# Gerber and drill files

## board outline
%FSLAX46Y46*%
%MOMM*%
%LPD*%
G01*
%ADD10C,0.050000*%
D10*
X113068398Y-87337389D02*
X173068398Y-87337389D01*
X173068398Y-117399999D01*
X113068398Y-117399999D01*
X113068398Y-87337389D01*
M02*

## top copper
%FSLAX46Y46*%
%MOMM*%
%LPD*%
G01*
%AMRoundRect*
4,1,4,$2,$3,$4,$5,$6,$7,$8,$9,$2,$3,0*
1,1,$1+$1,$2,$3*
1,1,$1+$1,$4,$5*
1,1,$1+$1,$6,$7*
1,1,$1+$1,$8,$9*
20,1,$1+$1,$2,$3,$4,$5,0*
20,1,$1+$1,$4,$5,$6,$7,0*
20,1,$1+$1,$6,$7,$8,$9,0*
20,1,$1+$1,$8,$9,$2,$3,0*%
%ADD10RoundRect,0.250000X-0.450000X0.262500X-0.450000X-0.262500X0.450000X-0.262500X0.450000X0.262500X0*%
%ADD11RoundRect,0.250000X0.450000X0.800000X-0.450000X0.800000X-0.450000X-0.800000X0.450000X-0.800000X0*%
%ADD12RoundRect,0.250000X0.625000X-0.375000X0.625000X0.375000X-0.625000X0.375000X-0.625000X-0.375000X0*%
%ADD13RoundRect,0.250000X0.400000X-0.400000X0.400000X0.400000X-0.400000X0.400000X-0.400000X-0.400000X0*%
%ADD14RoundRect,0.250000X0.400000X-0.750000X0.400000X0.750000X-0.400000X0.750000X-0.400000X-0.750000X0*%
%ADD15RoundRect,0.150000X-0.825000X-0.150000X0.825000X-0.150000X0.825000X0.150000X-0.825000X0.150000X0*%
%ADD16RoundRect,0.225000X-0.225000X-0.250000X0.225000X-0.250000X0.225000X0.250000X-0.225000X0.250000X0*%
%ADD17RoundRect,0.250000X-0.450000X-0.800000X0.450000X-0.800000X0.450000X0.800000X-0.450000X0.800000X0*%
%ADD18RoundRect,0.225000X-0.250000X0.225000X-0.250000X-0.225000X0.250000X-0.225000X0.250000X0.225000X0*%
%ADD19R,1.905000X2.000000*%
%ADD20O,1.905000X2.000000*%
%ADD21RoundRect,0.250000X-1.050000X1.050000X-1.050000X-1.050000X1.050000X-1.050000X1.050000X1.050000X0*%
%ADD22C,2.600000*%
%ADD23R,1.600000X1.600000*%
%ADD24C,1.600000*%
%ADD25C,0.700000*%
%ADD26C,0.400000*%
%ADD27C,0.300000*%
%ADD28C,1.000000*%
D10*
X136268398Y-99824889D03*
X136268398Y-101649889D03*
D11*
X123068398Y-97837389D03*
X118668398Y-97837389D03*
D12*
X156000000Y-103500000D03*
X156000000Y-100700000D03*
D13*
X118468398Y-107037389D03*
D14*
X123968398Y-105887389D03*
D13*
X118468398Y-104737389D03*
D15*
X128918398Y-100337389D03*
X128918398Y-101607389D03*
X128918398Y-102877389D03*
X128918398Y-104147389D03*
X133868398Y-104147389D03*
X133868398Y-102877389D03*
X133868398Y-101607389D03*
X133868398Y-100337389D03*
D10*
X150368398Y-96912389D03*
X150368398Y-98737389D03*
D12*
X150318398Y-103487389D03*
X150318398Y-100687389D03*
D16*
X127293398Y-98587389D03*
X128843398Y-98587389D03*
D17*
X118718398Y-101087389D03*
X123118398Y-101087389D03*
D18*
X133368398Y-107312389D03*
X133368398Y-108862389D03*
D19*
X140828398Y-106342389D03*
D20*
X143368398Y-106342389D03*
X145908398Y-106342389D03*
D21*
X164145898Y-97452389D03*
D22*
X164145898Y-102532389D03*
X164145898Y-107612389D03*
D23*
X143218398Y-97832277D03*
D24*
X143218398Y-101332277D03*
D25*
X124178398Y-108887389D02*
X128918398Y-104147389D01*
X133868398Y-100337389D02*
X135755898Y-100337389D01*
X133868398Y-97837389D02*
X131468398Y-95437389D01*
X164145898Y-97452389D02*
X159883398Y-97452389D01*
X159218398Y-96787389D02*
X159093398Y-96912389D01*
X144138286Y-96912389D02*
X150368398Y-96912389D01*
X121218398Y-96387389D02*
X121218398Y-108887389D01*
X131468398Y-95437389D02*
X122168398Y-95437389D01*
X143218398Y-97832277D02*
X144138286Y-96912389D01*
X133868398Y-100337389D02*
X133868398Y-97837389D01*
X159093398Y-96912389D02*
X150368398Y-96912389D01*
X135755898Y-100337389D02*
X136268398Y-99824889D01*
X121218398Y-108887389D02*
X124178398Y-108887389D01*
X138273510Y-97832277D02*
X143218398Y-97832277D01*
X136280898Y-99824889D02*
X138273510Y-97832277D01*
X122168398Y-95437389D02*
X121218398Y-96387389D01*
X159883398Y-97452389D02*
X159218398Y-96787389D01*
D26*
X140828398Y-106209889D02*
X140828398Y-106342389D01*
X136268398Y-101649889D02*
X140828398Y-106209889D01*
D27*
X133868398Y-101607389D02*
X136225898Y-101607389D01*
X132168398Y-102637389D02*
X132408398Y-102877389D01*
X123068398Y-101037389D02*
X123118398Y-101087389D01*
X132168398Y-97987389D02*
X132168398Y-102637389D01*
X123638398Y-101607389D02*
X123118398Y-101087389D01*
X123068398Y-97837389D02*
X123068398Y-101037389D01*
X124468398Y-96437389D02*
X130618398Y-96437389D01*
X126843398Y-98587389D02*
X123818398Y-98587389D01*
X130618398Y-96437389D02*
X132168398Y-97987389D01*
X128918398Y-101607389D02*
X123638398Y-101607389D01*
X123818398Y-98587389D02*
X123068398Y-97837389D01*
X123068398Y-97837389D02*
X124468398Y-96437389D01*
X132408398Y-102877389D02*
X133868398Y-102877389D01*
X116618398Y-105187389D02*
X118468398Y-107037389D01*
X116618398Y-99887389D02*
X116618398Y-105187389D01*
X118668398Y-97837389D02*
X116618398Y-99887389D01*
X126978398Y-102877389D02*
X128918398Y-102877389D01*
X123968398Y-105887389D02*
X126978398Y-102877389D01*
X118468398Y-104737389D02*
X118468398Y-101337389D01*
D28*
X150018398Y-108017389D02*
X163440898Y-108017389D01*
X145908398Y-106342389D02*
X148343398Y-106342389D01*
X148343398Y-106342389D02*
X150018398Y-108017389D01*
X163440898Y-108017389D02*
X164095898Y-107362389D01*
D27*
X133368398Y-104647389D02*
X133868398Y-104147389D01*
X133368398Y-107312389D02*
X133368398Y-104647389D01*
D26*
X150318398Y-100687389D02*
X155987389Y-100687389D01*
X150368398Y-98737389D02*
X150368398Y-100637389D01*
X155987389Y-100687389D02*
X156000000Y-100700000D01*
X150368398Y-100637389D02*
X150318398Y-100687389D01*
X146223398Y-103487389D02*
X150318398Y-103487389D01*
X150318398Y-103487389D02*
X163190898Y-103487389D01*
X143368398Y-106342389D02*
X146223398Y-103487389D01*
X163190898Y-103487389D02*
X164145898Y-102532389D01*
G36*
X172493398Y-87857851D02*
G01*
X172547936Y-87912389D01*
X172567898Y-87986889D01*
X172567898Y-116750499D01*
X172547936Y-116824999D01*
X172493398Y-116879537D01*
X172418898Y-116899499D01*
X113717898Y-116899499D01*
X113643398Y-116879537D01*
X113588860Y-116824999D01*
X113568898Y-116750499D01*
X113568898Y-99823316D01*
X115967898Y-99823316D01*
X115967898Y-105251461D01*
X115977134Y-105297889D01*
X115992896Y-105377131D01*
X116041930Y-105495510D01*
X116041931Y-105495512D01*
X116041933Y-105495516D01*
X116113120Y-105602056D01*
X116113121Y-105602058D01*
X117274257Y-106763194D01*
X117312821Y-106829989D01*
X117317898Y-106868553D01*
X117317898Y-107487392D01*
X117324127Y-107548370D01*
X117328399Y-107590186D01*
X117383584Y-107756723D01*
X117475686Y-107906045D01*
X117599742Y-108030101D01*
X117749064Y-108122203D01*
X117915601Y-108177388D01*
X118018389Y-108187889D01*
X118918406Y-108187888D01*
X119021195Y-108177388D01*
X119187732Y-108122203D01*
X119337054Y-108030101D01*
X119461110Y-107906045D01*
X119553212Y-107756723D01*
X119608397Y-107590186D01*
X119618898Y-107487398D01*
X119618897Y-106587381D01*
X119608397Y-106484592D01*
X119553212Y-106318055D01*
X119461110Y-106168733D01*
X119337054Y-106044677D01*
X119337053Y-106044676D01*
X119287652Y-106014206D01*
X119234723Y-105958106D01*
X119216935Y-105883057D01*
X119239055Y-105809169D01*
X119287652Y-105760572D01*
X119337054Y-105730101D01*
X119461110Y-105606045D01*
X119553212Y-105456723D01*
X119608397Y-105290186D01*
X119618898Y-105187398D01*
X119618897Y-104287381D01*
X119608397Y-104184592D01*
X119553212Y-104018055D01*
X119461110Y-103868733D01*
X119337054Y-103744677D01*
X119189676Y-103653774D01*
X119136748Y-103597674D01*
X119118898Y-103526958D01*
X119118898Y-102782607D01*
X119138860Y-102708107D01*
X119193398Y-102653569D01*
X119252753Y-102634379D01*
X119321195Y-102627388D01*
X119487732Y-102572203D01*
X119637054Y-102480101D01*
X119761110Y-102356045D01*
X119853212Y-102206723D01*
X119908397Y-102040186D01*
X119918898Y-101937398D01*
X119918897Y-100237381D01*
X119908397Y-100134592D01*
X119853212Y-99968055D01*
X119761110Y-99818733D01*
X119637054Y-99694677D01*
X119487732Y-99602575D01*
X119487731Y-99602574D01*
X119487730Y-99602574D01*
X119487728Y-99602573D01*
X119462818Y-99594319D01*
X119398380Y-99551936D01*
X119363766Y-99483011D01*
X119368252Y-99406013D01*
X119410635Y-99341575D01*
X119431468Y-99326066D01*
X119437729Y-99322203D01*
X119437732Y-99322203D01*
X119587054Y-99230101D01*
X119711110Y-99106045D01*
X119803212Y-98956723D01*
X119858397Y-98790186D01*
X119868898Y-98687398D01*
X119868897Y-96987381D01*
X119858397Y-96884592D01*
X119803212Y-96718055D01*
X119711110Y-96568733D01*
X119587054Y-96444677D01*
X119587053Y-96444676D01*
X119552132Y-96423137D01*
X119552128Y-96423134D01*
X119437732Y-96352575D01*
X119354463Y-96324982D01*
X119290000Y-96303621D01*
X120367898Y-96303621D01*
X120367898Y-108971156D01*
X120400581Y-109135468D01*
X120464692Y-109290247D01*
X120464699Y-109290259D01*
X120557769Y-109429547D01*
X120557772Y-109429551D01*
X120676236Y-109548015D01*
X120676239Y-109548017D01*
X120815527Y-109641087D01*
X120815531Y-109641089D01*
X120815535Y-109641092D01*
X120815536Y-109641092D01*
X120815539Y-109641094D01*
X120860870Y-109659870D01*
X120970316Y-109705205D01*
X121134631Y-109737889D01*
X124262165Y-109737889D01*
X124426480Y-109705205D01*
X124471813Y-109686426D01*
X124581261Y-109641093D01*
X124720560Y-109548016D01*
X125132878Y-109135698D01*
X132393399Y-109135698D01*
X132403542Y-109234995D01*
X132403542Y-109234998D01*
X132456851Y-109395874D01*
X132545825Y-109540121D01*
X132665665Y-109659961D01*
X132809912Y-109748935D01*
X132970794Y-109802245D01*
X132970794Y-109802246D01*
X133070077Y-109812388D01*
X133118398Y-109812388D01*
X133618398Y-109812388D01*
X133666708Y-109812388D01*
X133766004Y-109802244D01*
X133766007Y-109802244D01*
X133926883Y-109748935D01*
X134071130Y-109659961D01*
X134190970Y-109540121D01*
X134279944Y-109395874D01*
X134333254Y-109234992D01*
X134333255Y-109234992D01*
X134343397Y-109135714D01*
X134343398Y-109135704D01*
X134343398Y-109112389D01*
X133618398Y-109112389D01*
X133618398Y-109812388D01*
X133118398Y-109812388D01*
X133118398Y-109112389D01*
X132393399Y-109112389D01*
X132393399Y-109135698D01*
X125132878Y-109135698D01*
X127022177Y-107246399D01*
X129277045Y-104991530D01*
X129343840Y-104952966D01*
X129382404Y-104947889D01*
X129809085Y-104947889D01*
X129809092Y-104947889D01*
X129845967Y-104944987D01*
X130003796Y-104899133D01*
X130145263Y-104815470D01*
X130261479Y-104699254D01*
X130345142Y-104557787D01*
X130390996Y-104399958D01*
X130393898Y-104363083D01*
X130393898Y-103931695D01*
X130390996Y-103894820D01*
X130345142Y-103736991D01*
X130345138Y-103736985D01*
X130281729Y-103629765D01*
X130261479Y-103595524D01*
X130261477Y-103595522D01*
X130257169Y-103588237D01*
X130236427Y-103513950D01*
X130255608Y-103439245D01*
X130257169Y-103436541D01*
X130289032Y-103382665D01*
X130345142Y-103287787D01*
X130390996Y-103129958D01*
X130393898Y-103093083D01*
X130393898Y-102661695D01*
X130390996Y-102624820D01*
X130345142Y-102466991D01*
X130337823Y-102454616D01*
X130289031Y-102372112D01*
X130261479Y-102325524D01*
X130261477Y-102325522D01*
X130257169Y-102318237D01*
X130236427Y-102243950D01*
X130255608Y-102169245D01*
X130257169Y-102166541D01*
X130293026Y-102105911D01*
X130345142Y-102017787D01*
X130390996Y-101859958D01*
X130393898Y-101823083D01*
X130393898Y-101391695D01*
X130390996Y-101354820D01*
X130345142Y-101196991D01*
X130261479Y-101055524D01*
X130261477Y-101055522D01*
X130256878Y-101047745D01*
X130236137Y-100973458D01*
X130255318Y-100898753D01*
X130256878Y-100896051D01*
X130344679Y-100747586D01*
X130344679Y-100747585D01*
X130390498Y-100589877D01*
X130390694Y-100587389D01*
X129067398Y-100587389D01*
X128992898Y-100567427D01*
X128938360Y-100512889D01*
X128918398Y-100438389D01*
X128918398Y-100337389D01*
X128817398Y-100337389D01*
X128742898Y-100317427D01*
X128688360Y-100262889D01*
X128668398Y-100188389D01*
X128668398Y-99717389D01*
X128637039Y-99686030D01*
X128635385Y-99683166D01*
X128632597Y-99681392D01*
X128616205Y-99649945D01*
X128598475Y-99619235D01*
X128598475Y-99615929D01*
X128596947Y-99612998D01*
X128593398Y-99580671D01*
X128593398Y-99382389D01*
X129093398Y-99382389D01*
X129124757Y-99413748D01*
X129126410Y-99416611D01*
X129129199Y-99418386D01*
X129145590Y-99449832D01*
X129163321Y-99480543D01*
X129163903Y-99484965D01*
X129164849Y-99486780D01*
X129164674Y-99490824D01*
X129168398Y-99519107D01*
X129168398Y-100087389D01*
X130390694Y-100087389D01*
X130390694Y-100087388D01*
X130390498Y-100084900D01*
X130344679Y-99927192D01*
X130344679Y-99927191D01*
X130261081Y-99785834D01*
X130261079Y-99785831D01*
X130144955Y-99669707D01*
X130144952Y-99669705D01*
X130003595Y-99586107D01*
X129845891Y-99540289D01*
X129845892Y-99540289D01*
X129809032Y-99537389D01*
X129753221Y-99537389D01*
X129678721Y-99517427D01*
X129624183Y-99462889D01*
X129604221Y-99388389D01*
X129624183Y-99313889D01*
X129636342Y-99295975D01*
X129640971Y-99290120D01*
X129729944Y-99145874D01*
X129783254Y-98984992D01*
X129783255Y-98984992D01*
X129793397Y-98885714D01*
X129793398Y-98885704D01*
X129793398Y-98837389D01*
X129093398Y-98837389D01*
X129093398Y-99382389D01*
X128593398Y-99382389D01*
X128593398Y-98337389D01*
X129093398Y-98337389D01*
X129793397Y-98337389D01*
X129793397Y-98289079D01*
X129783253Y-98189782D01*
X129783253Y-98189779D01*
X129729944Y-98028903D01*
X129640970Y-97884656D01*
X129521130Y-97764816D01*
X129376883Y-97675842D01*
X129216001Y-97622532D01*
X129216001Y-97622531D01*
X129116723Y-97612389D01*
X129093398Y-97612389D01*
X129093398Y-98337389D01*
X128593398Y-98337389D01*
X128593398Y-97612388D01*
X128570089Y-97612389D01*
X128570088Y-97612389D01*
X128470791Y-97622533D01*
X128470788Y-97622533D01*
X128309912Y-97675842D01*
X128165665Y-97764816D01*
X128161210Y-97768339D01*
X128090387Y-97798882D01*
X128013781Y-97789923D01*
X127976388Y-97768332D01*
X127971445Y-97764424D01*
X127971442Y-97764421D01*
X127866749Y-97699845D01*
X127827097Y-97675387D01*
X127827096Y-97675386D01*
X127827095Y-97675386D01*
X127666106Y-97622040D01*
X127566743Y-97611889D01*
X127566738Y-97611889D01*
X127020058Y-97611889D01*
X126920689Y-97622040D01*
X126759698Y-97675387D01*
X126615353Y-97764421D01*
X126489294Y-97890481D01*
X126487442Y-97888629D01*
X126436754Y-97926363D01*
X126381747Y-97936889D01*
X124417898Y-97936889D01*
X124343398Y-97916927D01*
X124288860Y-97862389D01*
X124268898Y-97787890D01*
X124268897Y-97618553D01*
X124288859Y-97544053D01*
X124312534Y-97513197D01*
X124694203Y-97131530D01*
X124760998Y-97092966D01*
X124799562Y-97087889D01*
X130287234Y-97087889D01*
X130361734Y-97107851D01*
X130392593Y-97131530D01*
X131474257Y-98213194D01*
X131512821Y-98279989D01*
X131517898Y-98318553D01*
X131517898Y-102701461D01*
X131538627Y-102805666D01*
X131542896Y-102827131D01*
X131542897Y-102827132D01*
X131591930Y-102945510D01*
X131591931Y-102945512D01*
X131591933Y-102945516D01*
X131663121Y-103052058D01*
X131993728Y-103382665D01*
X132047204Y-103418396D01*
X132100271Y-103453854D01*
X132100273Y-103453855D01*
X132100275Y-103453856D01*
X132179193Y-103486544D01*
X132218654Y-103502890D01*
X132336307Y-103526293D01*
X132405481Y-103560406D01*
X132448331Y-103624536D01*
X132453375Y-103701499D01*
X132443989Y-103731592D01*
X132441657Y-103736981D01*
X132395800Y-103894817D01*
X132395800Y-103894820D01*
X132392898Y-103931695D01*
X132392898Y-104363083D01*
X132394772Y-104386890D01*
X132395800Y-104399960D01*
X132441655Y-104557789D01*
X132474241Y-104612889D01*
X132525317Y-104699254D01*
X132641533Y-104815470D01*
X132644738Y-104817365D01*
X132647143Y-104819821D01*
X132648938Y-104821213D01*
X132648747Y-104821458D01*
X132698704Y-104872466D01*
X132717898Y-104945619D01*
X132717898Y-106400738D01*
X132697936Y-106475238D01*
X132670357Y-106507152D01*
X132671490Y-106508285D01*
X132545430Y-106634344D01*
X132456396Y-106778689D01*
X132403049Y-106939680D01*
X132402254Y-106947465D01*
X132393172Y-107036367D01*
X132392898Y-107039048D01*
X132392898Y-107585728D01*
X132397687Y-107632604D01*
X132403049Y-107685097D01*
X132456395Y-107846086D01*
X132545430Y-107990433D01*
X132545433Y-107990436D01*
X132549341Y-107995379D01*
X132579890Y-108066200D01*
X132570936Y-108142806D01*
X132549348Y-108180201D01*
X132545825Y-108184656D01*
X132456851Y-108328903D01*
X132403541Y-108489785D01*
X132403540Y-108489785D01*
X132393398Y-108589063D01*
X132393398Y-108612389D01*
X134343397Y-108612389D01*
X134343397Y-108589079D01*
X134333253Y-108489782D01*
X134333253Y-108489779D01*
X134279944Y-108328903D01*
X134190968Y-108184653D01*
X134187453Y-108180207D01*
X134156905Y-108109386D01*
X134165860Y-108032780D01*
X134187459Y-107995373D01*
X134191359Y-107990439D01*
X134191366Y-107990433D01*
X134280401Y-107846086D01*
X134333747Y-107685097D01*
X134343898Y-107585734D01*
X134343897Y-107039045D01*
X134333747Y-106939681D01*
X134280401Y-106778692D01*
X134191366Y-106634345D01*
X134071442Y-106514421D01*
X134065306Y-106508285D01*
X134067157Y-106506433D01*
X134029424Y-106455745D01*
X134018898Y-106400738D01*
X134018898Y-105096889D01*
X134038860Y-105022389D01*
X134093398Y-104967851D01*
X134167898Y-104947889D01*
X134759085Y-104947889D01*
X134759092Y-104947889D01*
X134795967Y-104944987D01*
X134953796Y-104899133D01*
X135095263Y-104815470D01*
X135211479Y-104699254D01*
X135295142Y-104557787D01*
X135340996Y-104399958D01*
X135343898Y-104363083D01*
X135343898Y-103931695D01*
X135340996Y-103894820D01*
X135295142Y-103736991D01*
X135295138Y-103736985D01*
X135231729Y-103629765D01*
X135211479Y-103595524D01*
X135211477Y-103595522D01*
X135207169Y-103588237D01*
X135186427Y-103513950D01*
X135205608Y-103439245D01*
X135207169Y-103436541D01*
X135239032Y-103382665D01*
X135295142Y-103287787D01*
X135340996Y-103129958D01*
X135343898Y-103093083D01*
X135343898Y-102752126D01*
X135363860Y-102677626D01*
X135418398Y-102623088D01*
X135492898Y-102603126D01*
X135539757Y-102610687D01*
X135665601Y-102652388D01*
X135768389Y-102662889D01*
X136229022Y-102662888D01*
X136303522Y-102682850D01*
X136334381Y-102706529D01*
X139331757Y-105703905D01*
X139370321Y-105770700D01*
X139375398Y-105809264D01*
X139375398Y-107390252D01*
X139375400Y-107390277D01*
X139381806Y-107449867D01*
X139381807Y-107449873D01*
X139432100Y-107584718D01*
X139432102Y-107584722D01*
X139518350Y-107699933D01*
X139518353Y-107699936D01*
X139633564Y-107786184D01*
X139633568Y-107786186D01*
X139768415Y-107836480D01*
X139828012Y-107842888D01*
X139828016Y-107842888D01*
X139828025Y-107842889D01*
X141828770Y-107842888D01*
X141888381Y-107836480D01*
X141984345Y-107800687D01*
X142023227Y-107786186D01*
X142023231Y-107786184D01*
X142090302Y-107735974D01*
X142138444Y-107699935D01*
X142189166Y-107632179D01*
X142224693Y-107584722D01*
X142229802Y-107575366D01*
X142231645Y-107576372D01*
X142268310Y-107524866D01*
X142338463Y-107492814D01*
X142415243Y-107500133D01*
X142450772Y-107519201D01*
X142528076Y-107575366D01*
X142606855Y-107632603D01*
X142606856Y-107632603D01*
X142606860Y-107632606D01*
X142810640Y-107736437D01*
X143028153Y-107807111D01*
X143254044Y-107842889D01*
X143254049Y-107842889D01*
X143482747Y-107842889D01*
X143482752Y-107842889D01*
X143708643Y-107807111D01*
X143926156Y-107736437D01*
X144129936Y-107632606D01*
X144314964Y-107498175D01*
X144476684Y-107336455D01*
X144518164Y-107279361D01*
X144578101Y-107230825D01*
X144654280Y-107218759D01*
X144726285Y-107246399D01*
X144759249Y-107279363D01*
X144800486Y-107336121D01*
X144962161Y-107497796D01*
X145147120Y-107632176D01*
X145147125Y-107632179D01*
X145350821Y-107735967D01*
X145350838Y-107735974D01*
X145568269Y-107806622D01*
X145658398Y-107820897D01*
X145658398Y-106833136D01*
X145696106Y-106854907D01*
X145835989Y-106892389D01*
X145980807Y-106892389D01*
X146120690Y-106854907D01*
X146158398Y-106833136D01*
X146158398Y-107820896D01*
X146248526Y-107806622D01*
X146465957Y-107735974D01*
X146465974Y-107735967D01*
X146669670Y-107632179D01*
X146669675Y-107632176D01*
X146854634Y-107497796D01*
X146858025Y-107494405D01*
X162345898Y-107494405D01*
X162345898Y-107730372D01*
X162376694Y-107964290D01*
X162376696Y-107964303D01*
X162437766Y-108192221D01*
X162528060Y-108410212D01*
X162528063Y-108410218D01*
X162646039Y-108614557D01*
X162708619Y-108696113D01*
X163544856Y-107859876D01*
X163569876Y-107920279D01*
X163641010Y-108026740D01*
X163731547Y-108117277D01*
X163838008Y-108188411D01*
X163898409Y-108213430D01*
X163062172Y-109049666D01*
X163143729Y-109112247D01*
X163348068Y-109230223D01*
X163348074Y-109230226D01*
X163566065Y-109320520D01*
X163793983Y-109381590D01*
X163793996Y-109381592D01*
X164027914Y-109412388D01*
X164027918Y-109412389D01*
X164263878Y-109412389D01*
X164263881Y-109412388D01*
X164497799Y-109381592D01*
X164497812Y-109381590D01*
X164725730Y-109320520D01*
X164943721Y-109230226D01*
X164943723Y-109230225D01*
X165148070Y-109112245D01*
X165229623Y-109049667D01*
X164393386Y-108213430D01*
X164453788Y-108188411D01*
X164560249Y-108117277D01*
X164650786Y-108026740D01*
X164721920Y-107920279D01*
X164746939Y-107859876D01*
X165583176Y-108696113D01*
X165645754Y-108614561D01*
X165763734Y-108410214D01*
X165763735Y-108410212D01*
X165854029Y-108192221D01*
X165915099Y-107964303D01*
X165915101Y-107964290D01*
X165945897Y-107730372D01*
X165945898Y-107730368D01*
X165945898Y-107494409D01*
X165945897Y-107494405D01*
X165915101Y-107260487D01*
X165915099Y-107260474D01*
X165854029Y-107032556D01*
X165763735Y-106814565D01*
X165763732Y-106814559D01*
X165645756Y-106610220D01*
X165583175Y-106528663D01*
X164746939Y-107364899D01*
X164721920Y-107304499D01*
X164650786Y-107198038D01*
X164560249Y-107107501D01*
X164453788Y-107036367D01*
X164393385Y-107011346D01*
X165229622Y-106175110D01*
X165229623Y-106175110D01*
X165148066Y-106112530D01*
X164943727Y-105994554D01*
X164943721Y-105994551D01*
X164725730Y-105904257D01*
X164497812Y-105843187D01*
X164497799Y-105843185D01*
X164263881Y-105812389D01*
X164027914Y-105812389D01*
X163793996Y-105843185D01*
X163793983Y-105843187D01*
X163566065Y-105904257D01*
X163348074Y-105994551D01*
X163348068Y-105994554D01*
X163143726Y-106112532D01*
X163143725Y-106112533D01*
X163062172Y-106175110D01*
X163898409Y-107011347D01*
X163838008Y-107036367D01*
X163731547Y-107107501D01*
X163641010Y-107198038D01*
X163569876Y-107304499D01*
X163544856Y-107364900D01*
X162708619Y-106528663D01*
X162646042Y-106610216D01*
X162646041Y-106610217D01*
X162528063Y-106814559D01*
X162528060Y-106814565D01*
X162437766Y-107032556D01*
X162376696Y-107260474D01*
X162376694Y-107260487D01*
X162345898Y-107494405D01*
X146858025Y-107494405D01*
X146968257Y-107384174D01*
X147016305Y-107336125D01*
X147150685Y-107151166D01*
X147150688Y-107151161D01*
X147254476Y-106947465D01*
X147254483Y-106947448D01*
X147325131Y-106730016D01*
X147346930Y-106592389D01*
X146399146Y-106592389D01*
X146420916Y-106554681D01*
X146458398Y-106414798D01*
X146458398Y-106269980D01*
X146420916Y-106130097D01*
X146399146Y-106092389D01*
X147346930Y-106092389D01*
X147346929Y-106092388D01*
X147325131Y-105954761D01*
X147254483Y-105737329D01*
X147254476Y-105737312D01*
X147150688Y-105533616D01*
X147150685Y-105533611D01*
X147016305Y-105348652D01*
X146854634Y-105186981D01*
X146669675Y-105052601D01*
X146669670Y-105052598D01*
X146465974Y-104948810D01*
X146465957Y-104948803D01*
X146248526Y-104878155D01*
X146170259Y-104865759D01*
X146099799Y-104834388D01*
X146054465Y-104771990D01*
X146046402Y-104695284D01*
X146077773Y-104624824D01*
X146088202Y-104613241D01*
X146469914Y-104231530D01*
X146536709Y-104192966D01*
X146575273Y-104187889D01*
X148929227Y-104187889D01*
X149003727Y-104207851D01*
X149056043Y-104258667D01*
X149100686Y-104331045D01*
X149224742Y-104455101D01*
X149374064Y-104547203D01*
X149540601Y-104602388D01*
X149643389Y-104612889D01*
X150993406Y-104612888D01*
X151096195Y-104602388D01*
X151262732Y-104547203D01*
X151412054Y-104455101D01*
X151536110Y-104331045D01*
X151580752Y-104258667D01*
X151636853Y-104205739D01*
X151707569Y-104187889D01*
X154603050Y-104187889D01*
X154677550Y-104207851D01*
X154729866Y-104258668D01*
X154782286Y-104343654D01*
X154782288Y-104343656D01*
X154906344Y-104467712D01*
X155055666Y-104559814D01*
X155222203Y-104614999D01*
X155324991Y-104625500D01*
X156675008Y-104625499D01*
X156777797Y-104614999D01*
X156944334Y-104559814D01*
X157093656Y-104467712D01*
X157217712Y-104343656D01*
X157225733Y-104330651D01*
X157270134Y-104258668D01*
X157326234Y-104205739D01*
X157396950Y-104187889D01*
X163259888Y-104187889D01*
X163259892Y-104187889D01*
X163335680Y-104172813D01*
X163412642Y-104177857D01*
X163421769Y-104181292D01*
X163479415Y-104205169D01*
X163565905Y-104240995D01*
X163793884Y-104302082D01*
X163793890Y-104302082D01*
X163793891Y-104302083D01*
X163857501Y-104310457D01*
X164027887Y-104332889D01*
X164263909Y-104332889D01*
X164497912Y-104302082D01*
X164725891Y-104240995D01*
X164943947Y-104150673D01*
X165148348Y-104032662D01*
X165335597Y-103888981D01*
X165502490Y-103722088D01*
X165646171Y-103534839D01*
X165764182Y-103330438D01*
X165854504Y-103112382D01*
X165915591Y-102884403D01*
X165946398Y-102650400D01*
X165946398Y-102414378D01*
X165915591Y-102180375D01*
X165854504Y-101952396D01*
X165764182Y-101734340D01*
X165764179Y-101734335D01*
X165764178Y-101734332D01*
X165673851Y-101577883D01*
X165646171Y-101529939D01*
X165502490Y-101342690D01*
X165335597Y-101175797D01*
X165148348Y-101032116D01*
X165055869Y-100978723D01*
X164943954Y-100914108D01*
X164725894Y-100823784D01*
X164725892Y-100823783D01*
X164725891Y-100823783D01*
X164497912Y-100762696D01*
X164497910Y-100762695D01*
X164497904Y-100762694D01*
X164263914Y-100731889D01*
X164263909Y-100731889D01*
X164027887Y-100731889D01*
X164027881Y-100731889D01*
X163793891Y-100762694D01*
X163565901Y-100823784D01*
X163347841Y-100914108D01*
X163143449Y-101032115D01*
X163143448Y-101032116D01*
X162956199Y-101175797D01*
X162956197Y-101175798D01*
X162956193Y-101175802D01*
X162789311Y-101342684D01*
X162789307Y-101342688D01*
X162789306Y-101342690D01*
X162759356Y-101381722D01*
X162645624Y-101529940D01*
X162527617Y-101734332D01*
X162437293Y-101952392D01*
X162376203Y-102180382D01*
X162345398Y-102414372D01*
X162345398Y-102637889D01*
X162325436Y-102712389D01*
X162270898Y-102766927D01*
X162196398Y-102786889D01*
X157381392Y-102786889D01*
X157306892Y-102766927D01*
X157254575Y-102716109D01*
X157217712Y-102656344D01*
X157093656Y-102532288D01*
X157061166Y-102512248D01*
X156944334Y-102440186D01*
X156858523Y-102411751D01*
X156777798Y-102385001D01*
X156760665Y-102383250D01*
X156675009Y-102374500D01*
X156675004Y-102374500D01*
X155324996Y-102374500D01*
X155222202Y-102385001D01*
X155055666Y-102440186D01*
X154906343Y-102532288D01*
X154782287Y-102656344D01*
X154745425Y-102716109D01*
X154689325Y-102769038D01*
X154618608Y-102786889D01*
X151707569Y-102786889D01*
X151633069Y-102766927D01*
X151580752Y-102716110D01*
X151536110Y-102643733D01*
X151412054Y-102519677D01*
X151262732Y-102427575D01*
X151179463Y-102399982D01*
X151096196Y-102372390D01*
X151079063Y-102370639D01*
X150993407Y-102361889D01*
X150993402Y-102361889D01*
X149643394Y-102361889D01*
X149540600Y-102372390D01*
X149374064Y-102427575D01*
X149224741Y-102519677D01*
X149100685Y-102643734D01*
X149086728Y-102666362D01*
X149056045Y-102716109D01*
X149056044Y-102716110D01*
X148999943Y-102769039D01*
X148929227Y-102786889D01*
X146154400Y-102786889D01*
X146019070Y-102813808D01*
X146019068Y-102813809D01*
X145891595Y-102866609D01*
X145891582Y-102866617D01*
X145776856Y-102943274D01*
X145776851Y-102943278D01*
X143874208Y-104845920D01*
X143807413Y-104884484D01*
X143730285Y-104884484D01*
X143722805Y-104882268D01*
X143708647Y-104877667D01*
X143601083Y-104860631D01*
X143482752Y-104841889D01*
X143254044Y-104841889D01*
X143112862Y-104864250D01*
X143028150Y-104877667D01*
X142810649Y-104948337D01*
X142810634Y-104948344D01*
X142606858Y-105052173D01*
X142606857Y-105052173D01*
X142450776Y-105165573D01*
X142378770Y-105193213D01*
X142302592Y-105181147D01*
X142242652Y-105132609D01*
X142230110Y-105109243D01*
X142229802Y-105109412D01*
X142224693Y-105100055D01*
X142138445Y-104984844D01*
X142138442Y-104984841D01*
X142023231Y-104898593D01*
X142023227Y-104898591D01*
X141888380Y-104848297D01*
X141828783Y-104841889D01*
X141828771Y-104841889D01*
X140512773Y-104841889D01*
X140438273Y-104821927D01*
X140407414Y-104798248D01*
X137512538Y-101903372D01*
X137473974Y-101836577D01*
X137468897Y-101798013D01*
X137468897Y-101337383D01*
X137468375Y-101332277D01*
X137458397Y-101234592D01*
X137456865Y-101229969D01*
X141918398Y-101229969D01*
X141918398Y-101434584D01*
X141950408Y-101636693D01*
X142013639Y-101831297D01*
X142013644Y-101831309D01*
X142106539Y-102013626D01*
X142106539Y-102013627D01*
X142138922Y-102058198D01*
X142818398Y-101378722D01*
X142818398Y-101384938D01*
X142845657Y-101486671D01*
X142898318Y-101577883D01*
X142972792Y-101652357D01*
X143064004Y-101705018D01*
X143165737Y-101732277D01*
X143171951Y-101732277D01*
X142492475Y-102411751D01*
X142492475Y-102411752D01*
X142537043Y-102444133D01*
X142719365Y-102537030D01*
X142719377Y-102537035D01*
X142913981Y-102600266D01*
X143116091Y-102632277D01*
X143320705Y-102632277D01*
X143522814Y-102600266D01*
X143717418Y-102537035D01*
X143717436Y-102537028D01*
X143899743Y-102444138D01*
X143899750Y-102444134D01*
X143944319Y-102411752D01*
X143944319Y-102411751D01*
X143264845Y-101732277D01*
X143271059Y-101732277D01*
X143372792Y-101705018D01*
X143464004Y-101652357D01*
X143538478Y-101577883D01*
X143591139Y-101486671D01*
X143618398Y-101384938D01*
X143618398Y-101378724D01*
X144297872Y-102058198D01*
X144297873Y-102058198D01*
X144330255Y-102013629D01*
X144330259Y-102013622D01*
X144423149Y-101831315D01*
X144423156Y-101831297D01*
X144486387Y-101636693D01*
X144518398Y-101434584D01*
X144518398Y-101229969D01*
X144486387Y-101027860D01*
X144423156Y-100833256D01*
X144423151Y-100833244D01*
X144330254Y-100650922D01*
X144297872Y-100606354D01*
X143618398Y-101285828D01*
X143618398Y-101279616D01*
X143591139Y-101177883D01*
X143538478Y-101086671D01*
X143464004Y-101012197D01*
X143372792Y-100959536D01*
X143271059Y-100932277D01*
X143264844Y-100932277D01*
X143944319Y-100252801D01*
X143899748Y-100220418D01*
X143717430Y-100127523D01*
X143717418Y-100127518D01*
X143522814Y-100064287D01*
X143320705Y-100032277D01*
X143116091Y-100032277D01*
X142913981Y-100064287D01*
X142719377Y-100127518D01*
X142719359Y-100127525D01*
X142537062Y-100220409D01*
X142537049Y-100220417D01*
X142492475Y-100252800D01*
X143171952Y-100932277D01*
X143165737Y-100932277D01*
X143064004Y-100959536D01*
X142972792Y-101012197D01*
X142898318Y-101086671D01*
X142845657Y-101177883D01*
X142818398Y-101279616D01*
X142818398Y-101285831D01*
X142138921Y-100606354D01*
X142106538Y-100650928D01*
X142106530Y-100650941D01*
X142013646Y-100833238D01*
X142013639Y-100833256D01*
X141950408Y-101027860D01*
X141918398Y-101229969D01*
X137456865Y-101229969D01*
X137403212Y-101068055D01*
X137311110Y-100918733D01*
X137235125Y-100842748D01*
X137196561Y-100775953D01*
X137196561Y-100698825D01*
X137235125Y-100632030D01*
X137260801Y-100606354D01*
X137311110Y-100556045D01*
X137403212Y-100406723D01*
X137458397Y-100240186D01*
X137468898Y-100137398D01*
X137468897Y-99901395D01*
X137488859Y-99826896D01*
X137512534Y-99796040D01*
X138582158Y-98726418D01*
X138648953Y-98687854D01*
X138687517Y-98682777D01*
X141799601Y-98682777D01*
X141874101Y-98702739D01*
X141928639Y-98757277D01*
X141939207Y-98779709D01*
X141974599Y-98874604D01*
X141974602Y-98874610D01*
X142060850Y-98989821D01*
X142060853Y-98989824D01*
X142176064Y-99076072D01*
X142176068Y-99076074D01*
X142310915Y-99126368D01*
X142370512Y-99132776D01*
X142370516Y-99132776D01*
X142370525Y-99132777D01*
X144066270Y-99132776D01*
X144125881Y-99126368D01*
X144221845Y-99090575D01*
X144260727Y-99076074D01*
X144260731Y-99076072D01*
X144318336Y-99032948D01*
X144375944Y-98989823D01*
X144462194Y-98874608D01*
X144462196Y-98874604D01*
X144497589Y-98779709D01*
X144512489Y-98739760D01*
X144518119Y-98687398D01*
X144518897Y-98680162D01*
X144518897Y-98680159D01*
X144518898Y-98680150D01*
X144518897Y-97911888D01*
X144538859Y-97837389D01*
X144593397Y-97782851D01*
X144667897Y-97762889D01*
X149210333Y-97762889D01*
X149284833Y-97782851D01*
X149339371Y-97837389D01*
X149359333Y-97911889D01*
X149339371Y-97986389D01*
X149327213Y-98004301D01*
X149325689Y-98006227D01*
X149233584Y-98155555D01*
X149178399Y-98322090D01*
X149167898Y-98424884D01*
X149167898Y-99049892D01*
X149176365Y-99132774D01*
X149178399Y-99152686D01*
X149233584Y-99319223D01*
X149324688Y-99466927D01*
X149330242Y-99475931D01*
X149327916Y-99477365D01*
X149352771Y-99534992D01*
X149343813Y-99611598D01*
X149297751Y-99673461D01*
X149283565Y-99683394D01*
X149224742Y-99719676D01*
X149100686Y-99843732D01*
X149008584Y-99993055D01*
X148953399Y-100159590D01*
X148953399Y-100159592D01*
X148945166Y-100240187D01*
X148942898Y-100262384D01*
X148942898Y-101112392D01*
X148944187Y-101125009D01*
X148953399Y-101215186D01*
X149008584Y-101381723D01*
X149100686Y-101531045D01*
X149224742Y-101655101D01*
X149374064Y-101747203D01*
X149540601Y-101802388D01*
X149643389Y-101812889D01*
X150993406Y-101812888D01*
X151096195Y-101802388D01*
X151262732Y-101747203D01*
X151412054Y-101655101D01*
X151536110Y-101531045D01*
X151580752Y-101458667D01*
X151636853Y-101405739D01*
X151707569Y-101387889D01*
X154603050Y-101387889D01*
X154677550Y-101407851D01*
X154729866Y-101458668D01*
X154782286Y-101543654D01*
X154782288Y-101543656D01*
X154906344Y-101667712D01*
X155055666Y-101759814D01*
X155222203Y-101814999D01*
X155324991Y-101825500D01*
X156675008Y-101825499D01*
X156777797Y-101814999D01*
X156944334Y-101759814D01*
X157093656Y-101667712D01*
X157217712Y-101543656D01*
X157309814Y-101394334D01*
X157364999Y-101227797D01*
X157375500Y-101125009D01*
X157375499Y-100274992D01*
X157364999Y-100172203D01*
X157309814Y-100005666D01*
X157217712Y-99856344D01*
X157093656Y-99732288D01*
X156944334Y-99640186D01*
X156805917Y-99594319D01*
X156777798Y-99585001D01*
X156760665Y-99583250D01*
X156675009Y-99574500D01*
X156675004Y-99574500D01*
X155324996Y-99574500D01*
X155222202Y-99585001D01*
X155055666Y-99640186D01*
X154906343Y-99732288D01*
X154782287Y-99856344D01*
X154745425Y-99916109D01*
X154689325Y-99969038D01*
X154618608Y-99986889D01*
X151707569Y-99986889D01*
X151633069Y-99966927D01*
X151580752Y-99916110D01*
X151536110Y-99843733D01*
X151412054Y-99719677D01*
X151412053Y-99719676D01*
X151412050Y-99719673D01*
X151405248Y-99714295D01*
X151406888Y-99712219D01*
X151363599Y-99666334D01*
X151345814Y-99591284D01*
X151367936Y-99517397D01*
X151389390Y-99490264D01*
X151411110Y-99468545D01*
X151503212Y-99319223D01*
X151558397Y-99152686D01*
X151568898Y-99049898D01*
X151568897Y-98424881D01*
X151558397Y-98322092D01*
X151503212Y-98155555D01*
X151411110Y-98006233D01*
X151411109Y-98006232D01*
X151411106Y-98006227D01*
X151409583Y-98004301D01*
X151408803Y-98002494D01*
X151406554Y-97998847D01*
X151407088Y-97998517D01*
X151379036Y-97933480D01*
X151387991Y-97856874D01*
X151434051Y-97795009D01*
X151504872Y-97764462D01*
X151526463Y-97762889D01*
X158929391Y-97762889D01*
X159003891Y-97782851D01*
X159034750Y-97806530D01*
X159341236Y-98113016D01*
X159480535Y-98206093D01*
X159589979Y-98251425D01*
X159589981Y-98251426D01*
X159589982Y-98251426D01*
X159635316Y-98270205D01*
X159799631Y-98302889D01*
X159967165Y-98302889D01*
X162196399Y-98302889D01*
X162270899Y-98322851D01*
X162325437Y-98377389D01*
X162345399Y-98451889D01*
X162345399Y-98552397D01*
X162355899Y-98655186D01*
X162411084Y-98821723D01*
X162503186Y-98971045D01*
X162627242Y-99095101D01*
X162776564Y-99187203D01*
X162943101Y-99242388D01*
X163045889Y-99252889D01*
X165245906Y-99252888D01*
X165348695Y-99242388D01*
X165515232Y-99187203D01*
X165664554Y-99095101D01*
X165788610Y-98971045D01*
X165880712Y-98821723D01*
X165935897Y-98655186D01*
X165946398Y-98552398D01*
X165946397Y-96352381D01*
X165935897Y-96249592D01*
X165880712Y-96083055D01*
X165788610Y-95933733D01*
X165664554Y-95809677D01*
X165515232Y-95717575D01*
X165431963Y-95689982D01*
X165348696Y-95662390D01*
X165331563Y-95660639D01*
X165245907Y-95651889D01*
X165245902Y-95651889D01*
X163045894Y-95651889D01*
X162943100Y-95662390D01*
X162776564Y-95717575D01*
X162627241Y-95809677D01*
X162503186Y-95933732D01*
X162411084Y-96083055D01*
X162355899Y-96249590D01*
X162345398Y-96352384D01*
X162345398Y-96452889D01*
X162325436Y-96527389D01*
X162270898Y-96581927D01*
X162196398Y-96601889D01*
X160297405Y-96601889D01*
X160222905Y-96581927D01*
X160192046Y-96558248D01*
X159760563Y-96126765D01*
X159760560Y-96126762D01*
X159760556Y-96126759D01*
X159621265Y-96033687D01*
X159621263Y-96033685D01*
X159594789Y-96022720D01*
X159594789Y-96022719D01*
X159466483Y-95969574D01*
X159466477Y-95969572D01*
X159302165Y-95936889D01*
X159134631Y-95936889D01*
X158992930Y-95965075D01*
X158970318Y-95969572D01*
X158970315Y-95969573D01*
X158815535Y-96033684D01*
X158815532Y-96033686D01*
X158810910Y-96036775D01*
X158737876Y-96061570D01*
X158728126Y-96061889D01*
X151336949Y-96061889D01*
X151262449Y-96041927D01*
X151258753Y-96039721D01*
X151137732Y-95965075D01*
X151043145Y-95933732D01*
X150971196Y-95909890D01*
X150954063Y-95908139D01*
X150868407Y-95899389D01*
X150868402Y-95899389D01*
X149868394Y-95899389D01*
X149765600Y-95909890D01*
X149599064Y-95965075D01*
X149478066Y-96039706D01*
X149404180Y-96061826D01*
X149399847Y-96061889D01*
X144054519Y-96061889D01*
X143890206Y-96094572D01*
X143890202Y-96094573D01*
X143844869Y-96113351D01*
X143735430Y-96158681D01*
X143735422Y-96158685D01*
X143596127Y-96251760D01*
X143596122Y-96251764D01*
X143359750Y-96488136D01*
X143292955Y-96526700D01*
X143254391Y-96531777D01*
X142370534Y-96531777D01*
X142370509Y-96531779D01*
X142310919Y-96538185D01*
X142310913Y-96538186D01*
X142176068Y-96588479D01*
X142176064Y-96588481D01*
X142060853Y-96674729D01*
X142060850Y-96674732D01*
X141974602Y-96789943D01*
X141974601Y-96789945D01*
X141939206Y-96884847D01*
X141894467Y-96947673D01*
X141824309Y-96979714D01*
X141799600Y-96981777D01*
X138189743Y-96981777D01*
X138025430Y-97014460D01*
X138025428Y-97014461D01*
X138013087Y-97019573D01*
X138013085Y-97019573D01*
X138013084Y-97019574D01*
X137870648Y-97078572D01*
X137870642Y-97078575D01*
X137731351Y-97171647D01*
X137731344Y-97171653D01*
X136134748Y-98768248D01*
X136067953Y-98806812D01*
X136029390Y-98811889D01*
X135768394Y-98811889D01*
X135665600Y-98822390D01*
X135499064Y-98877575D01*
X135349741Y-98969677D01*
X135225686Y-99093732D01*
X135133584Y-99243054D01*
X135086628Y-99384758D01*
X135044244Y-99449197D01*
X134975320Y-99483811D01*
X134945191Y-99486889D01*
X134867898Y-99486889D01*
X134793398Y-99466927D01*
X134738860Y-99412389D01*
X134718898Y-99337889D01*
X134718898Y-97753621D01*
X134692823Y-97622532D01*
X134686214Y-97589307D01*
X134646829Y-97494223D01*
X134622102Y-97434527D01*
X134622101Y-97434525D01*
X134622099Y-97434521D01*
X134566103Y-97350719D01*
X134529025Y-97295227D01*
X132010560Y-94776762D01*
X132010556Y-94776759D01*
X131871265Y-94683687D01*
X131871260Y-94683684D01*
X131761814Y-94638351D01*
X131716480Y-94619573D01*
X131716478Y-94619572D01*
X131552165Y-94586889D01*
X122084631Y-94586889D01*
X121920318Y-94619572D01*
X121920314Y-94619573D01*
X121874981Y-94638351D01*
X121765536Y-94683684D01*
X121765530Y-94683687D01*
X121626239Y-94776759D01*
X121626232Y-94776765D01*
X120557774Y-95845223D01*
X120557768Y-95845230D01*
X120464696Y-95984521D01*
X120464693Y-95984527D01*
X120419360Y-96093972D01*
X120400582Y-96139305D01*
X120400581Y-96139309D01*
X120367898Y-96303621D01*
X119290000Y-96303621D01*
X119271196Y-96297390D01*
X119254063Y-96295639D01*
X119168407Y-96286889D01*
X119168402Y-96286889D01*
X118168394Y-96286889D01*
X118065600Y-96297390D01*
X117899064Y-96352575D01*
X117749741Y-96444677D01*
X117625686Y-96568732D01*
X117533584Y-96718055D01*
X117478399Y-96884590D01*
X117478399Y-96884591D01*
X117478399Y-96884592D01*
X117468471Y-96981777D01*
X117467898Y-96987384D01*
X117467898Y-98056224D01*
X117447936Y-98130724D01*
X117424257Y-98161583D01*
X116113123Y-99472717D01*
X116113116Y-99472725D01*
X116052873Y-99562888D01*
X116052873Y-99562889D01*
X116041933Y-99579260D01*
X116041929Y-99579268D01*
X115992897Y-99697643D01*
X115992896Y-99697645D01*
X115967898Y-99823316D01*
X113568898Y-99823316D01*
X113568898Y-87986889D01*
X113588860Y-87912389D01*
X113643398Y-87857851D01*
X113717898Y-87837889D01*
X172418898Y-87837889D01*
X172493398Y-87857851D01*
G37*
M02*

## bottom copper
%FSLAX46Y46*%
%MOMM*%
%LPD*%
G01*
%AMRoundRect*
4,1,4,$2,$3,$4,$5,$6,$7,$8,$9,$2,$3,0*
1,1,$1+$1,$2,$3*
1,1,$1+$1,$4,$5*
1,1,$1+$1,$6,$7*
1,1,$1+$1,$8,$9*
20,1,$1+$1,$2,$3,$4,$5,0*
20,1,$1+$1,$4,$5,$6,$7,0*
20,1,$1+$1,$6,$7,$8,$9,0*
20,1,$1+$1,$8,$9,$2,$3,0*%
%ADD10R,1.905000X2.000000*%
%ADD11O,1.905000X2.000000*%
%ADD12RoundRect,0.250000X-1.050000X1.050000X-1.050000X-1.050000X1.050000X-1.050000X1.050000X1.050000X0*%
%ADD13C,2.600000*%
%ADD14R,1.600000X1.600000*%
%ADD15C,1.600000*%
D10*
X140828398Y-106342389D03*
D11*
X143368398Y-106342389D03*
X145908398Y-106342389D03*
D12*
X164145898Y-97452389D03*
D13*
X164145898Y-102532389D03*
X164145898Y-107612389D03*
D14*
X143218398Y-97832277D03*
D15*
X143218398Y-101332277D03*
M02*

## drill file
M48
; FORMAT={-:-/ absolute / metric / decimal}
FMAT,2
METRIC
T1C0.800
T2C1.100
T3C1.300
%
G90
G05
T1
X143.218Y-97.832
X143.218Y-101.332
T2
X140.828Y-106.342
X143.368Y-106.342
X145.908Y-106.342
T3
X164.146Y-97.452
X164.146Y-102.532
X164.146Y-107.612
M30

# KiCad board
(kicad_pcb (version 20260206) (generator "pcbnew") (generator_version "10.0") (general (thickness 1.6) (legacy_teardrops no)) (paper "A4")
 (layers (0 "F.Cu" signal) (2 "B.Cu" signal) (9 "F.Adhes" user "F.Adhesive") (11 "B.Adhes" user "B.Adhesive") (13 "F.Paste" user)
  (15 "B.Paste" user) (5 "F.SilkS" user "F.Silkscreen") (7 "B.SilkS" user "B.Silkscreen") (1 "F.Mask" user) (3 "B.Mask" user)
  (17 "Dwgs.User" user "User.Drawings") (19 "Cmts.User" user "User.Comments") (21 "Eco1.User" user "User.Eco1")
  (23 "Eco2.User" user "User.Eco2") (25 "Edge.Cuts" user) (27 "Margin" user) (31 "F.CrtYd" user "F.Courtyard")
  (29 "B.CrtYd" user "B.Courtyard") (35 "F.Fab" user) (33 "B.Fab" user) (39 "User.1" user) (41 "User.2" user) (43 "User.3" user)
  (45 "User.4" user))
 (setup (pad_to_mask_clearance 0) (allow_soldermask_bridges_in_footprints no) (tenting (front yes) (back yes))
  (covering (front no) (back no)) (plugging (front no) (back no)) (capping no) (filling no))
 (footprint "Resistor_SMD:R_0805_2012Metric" (layer "F.Cu") (at 136.268398 100.737389 -90)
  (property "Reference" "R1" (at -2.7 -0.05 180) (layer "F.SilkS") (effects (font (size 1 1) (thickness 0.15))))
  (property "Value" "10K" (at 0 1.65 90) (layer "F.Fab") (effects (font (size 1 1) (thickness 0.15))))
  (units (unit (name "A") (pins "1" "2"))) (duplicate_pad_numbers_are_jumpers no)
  (pad "1" smd roundrect (at -0.9125 0 270) (size 1.025 1.4) (layers "F.Cu" "F.Mask" "F.Paste") (roundrect_rratio 0.243902) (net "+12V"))
  (pad "2" smd roundrect (at 0.9125 0 270) (size 1.025 1.4) (layers "F.Cu" "F.Mask" "F.Paste") (roundrect_rratio 0.243902)
   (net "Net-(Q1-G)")))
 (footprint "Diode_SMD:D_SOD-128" (layer "F.Cu") (at 120.868398 97.837389 180)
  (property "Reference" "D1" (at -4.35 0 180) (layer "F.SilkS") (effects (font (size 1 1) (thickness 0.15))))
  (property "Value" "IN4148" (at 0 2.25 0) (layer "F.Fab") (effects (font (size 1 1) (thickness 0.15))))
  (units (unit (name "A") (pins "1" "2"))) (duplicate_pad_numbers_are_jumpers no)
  (pad "1" smd roundrect (at -2.2 0 180) (size 1.4 2.1) (layers "F.Cu" "F.Mask" "F.Paste") (roundrect_rratio 0.1785714286) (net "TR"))
  (pad "2" smd roundrect (at 2.2 0 180) (size 1.4 2.1) (layers "F.Cu" "F.Mask" "F.Paste") (roundrect_rratio 0.1785714286) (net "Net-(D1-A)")))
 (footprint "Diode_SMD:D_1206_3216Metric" (layer "F.Cu") (at 156 102.1 90)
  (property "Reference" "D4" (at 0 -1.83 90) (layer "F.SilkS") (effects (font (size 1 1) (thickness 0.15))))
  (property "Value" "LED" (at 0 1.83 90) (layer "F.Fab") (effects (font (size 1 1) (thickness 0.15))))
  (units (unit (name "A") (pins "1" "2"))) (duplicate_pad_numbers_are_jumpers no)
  (pad "1" smd roundrect (at -1.4 0 90) (size 1.25 1.75) (layers "F.Cu" "F.Mask" "F.Paste") (roundrect_rratio 0.2) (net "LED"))
  (pad "2" smd roundrect (at 1.4 0 90) (size 1.25 1.75) (layers "F.Cu" "F.Mask" "F.Paste") (roundrect_rratio 0.2) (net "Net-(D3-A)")))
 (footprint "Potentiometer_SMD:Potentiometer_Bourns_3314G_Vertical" (layer "F.Cu") (at 121.218398 105.887389 90)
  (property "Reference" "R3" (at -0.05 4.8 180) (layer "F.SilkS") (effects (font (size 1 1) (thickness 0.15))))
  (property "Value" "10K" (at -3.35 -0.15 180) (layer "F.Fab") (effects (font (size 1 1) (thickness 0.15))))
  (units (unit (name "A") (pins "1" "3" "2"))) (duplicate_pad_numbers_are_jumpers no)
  (pad "1" smd roundrect (at -1.15 -2.75 90) (size 1.3 1.3) (layers "F.Cu" "F.Mask" "F.Paste") (roundrect_rratio 0.1923076923)
   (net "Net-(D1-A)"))
  (pad "2" smd roundrect (at 0 2.75 90) (size 2 1.3) (layers "F.Cu" "F.Mask" "F.Paste") (roundrect_rratio 0.1923076923) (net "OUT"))
  (pad "3" smd roundrect (at 1.15 -2.75 90) (size 1.3 1.3) (layers "F.Cu" "F.Mask" "F.Paste") (roundrect_rratio 0.1923076923)
   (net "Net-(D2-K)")))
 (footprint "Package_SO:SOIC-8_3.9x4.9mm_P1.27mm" (layer "F.Cu") (at 131.393398 102.242389)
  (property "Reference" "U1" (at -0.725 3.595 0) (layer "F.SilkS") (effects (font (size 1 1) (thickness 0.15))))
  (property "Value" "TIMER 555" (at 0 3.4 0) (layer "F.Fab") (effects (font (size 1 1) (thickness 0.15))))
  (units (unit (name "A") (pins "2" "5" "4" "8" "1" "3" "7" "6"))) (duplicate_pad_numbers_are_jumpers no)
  (pad "1" smd roundrect (at -2.475 -1.905) (size 1.95 0.6) (layers "F.Cu" "F.Mask" "F.Paste") (roundrect_rratio 0.25) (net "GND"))
  (pad "2" smd roundrect (at -2.475 -0.635) (size 1.95 0.6) (layers "F.Cu" "F.Mask" "F.Paste") (roundrect_rratio 0.25) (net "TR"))
  (pad "3" smd roundrect (at -2.475 0.635) (size 1.95 0.6) (layers "F.Cu" "F.Mask" "F.Paste") (roundrect_rratio 0.25) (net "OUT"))
  (pad "4" smd roundrect (at -2.475 1.905) (size 1.95 0.6) (layers "F.Cu" "F.Mask" "F.Paste") (roundrect_rratio 0.25) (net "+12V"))
  (pad "5" smd roundrect (at 2.475 1.905) (size 1.95 0.6) (layers "F.Cu" "F.Mask" "F.Paste") (roundrect_rratio 0.25) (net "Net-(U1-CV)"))
  (pad "6" smd roundrect (at 2.475 0.635) (size 1.95 0.6) (layers "F.Cu" "F.Mask" "F.Paste") (roundrect_rratio 0.25) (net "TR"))
  (pad "7" smd roundrect (at 2.475 -0.635) (size 1.95 0.6) (layers "F.Cu" "F.Mask" "F.Paste") (roundrect_rratio 0.25) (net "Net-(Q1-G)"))
  (pad "8" smd roundrect (at 2.475 -1.905) (size 1.95 0.6) (layers "F.Cu" "F.Mask" "F.Paste") (roundrect_rratio 0.25) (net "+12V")))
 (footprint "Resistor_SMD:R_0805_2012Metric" (layer "F.Cu") (at 150.368398 97.824889 -90)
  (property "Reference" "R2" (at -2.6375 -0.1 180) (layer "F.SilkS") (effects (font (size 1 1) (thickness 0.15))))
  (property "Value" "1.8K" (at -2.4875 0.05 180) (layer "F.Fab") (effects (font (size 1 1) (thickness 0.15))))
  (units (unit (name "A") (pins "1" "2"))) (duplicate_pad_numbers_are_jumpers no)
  (pad "1" smd roundrect (at -0.9125 0 270) (size 1.025 1.4) (layers "F.Cu" "F.Mask" "F.Paste") (roundrect_rratio 0.243902) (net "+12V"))
  (pad "2" smd roundrect (at 0.9125 0 270) (size 1.025 1.4) (layers "F.Cu" "F.Mask" "F.Paste") (roundrect_rratio 0.243902)
   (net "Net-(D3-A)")))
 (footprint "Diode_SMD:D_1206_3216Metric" (layer "F.Cu") (at 150.318398 102.087389 90)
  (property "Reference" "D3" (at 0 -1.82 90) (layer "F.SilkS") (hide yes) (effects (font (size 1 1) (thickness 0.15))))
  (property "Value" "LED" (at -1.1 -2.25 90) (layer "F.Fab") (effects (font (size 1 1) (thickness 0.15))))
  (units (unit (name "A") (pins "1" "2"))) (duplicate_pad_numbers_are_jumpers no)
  (pad "1" smd roundrect (at -1.4 0 90) (size 1.25 1.75) (layers "F.Cu" "F.Mask" "F.Paste") (roundrect_rratio 0.2) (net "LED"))
  (pad "2" smd roundrect (at 1.4 0 90) (size 1.25 1.75) (layers "F.Cu" "F.Mask" "F.Paste") (roundrect_rratio 0.2) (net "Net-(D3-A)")))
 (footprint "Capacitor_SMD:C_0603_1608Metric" (layer "F.Cu") (at 128.068398 98.587389)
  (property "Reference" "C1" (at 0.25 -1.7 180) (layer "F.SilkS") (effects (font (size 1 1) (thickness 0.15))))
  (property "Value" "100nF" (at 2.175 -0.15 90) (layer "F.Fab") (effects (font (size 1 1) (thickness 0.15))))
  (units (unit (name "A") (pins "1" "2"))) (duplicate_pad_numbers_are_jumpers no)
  (pad "1" smd roundrect (at -0.775 0) (size 0.9 0.95) (layers "F.Cu" "F.Mask" "F.Paste") (roundrect_rratio 0.25) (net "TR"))
  (pad "2" smd roundrect (at 0.775 0) (size 0.9 0.95) (layers "F.Cu" "F.Mask" "F.Paste") (roundrect_rratio 0.25) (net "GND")))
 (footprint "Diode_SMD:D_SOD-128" (layer "F.Cu") (at 120.918398 101.087389)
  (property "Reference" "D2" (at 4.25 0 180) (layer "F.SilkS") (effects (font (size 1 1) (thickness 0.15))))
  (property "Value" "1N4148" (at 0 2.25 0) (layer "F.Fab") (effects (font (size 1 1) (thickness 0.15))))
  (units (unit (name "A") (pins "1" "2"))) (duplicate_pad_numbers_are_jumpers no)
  (pad "1" smd roundrect (at -2.2 0) (size 1.4 2.1) (layers "F.Cu" "F.Mask" "F.Paste") (roundrect_rratio 0.1785714286) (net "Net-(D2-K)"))
  (pad "2" smd roundrect (at 2.2 0) (size 1.4 2.1) (layers "F.Cu" "F.Mask" "F.Paste") (roundrect_rratio 0.1785714286) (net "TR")))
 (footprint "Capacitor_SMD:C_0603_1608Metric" (layer "F.Cu") (at 133.368398 108.087389 -90)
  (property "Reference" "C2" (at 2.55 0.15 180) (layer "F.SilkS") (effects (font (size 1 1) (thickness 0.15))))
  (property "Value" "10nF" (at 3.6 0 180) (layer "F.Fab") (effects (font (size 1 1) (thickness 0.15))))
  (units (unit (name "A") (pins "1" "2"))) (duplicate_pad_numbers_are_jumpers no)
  (pad "1" smd roundrect (at -0.775 0 270) (size 0.9 0.95) (layers "F.Cu" "F.Mask" "F.Paste") (roundrect_rratio 0.25) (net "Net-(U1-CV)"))
  (pad "2" smd roundrect (at 0.775 0 270) (size 0.9 0.95) (layers "F.Cu" "F.Mask" "F.Paste") (roundrect_rratio 0.25) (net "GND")))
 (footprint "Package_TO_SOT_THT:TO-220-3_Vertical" (layer "B.Cu") (at 140.828398 106.342389)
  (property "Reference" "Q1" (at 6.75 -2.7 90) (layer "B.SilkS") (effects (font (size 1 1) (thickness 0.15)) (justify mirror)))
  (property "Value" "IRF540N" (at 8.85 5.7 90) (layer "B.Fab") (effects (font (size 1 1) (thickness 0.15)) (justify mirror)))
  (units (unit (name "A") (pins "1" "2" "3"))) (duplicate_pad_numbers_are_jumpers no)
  (pad "1" thru_hole rect (at 0 0) (size 1.905 2) (drill 1.1) (layers "*.Cu" "*.Mask") (remove_unused_layers no) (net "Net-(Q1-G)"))
  (pad "2" thru_hole oval (at 2.54 0) (size 1.905 2) (drill 1.1) (layers "*.Cu" "*.Mask") (remove_unused_layers no) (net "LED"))
  (pad "3" thru_hole oval (at 5.08 0) (size 1.905 2) (drill 1.1) (layers "*.Cu" "*.Mask") (remove_unused_layers no) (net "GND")))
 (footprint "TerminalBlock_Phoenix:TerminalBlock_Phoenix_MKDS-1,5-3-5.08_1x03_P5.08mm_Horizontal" (layer "B.Cu")
  (at 164.145898 97.452389 -90)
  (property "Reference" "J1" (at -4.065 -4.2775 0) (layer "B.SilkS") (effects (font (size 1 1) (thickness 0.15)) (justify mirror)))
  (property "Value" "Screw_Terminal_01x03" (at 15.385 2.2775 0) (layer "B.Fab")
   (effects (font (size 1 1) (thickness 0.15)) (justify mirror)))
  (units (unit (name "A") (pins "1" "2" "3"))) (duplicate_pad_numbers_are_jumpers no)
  (pad "1" thru_hole roundrect (at 0 0 270) (size 2.6 2.6) (drill 1.3) (layers "*.Cu" "*.Mask") (remove_unused_layers no)
   (roundrect_rratio 0.096154) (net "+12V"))
  (pad "2" thru_hole circle (at 5.08 0 270) (size 2.6 2.6) (drill 1.3) (layers "*.Cu" "*.Mask") (remove_unused_layers no) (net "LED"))
  (pad "3" thru_hole circle (at 10.16 0 270) (size 2.6 2.6) (drill 1.3) (layers "*.Cu" "*.Mask") (remove_unused_layers no) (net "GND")))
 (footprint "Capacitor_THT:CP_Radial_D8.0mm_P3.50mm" (layer "B.Cu") (at 143.218398 97.832277 -90)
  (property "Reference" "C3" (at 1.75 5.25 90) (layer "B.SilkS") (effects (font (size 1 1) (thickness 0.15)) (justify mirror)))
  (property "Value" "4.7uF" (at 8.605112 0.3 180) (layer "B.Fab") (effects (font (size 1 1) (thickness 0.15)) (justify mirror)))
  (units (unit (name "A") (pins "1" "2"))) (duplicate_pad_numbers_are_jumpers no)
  (pad "1" thru_hole rect (at 0 0 270) (size 1.6 1.6) (drill 0.8) (layers "*.Cu" "*.Mask") (remove_unused_layers no) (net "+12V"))
  (pad "2" thru_hole circle (at 3.5 0 270) (size 1.6 1.6) (drill 0.8) (layers "*.Cu" "*.Mask") (remove_unused_layers no) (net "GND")))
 (gr_rect (start 113.068398 87.337389) (end 173.068398 117.399999) (stroke (width 0.05) (type default)) (fill no) (layer "Edge.Cuts"))
 (segment (start 124.178398 108.887389) (end 128.918398 104.147389) (width 0.7) (layer "F.Cu") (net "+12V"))
 (segment (start 133.868398 100.337389) (end 135.755898 100.337389) (width 0.7) (layer "F.Cu") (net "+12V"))
 (segment (start 133.868398 97.837389) (end 131.468398 95.437389) (width 0.7) (layer "F.Cu") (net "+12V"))
 (segment (start 164.145898 97.452389) (end 159.883398 97.452389) (width 0.7) (layer "F.Cu") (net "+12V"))
 (segment (start 159.218398 96.787389) (end 159.093398 96.912389) (width 0.7) (layer "F.Cu") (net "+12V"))
 (segment (start 144.138286 96.912389) (end 150.368398 96.912389) (width 0.7) (layer "F.Cu") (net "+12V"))
 (segment (start 121.218398 96.387389) (end 121.218398 108.887389) (width 0.7) (layer "F.Cu") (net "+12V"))
 (segment (start 131.468398 95.437389) (end 122.168398 95.437389) (width 0.7) (layer "F.Cu") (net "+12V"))
 (segment (start 143.218398 97.832277) (end 144.138286 96.912389) (width 0.7) (layer "F.Cu") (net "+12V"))
 (segment (start 133.868398 100.337389) (end 133.868398 97.837389) (width 0.7) (layer "F.Cu") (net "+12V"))
 (segment (start 159.093398 96.912389) (end 150.368398 96.912389) (width 0.7) (layer "F.Cu") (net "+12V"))
 (segment (start 135.755898 100.337389) (end 136.268398 99.824889) (width 0.7) (layer "F.Cu") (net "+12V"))
 (segment (start 121.218398 108.887389) (end 124.178398 108.887389) (width 0.7) (layer "F.Cu") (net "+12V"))
 (segment (start 138.27351 97.832277) (end 143.218398 97.832277) (width 0.7) (layer "F.Cu") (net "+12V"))
 (segment (start 136.280898 99.824889) (end 138.27351 97.832277) (width 0.7) (layer "F.Cu") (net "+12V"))
 (segment (start 122.168398 95.437389) (end 121.218398 96.387389) (width 0.7) (layer "F.Cu") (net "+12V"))
 (segment (start 159.883398 97.452389) (end 159.218398 96.787389) (width 0.7) (layer "F.Cu") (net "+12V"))
 (segment (start 140.828398 106.209889) (end 140.828398 106.342389) (width 0.4) (layer "F.Cu") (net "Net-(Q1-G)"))
 (segment (start 136.268398 101.649889) (end 140.828398 106.209889) (width 0.4) (layer "F.Cu") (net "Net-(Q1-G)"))
 (segment (start 133.868398 101.607389) (end 136.225898 101.607389) (width 0.3) (layer "F.Cu") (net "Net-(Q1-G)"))
 (segment (start 132.168398 102.637389) (end 132.408398 102.877389) (width 0.3) (layer "F.Cu") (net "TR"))
 (segment (start 123.068398 101.037389) (end 123.118398 101.087389) (width 0.3) (layer "F.Cu") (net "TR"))
 (segment (start 132.168398 97.987389) (end 132.168398 102.637389) (width 0.3) (layer "F.Cu") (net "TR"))
 (segment (start 123.638398 101.607389) (end 123.118398 101.087389) (width 0.3) (layer "F.Cu") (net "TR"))
 (segment (start 123.068398 97.837389) (end 123.068398 101.037389) (width 0.3) (layer "F.Cu") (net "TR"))
 (segment (start 124.468398 96.437389) (end 130.618398 96.437389) (width 0.3) (layer "F.Cu") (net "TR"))
 (segment (start 126.843398 98.587389) (end 123.818398 98.587389) (width 0.3) (layer "F.Cu") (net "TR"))
 (segment (start 130.618398 96.437389) (end 132.168398 97.987389) (width 0.3) (layer "F.Cu") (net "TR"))
 (segment (start 128.918398 101.607389) (end 123.638398 101.607389) (width 0.3) (layer "F.Cu") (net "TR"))
 (segment (start 123.818398 98.587389) (end 123.068398 97.837389) (width 0.3) (layer "F.Cu") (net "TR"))
 (segment (start 123.068398 97.837389) (end 124.468398 96.437389) (width 0.3) (layer "F.Cu") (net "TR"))
 (segment (start 132.408398 102.877389) (end 133.868398 102.877389) (width 0.3) (layer "F.Cu") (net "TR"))
 (segment (start 116.618398 105.187389) (end 118.468398 107.037389) (width 0.3) (layer "F.Cu") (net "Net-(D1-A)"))
 (segment (start 116.618398 99.887389) (end 116.618398 105.187389) (width 0.3) (layer "F.Cu") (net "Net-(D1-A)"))
 (segment (start 118.668398 97.837389) (end 116.618398 99.887389) (width 0.3) (layer "F.Cu") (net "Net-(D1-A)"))
 (segment (start 126.978398 102.877389) (end 128.918398 102.877389) (width 0.3) (layer "F.Cu") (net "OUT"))
 (segment (start 123.968398 105.887389) (end 126.978398 102.877389) (width 0.3) (layer "F.Cu") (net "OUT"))
 (segment (start 118.468398 104.737389) (end 118.468398 101.337389) (width 0.3) (layer "F.Cu") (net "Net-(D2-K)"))
 (segment (start 150.018398 108.017389) (end 163.440898 108.017389) (width 1) (layer "F.Cu") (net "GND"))
 (segment (start 145.908398 106.342389) (end 148.343398 106.342389) (width 1) (layer "F.Cu") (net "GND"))
 (segment (start 148.343398 106.342389) (end 150.018398 108.017389) (width 1) (layer "F.Cu") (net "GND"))
 (segment (start 163.440898 108.017389) (end 164.095898 107.362389) (width 1) (layer "F.Cu") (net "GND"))
 (segment (start 133.368398 104.647389) (end 133.868398 104.147389) (width 0.3) (layer "F.Cu") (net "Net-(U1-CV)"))
 (segment (start 133.368398 107.312389) (end 133.368398 104.647389) (width 0.3) (layer "F.Cu") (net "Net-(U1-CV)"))
 (segment (start 150.318398 100.687389) (end 155.987389 100.687389) (width 0.4) (layer "F.Cu") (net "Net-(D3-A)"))
 (segment (start 150.368398 98.737389) (end 150.368398 100.637389) (width 0.4) (layer "F.Cu") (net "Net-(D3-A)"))
 (segment (start 155.987389 100.687389) (end 156 100.7) (width 0.4) (layer "F.Cu") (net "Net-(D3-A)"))
 (segment (start 150.368398 100.637389) (end 150.318398 100.687389) (width 0.4) (layer "F.Cu") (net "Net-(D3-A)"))
 (segment (start 146.223398 103.487389) (end 150.318398 103.487389) (width 0.4) (layer "F.Cu") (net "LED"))
 (segment (start 150.318398 103.487389) (end 163.190898 103.487389) (width 0.4) (layer "F.Cu") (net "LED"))
 (segment (start 143.368398 106.342389) (end 146.223398 103.487389) (width 0.4) (layer "F.Cu") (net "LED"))
 (segment (start 163.190898 103.487389) (end 164.145898 102.532389) (width 0.4) (layer "F.Cu") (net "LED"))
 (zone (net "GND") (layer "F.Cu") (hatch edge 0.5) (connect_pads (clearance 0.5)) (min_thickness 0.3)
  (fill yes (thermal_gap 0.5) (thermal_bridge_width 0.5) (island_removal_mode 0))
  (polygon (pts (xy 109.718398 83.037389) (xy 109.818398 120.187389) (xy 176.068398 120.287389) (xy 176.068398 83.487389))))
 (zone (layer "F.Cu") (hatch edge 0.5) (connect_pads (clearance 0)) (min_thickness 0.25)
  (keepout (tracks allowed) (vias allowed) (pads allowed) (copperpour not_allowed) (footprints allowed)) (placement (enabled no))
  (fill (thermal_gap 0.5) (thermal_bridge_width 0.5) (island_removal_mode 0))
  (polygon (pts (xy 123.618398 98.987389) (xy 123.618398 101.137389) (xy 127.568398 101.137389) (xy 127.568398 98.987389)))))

